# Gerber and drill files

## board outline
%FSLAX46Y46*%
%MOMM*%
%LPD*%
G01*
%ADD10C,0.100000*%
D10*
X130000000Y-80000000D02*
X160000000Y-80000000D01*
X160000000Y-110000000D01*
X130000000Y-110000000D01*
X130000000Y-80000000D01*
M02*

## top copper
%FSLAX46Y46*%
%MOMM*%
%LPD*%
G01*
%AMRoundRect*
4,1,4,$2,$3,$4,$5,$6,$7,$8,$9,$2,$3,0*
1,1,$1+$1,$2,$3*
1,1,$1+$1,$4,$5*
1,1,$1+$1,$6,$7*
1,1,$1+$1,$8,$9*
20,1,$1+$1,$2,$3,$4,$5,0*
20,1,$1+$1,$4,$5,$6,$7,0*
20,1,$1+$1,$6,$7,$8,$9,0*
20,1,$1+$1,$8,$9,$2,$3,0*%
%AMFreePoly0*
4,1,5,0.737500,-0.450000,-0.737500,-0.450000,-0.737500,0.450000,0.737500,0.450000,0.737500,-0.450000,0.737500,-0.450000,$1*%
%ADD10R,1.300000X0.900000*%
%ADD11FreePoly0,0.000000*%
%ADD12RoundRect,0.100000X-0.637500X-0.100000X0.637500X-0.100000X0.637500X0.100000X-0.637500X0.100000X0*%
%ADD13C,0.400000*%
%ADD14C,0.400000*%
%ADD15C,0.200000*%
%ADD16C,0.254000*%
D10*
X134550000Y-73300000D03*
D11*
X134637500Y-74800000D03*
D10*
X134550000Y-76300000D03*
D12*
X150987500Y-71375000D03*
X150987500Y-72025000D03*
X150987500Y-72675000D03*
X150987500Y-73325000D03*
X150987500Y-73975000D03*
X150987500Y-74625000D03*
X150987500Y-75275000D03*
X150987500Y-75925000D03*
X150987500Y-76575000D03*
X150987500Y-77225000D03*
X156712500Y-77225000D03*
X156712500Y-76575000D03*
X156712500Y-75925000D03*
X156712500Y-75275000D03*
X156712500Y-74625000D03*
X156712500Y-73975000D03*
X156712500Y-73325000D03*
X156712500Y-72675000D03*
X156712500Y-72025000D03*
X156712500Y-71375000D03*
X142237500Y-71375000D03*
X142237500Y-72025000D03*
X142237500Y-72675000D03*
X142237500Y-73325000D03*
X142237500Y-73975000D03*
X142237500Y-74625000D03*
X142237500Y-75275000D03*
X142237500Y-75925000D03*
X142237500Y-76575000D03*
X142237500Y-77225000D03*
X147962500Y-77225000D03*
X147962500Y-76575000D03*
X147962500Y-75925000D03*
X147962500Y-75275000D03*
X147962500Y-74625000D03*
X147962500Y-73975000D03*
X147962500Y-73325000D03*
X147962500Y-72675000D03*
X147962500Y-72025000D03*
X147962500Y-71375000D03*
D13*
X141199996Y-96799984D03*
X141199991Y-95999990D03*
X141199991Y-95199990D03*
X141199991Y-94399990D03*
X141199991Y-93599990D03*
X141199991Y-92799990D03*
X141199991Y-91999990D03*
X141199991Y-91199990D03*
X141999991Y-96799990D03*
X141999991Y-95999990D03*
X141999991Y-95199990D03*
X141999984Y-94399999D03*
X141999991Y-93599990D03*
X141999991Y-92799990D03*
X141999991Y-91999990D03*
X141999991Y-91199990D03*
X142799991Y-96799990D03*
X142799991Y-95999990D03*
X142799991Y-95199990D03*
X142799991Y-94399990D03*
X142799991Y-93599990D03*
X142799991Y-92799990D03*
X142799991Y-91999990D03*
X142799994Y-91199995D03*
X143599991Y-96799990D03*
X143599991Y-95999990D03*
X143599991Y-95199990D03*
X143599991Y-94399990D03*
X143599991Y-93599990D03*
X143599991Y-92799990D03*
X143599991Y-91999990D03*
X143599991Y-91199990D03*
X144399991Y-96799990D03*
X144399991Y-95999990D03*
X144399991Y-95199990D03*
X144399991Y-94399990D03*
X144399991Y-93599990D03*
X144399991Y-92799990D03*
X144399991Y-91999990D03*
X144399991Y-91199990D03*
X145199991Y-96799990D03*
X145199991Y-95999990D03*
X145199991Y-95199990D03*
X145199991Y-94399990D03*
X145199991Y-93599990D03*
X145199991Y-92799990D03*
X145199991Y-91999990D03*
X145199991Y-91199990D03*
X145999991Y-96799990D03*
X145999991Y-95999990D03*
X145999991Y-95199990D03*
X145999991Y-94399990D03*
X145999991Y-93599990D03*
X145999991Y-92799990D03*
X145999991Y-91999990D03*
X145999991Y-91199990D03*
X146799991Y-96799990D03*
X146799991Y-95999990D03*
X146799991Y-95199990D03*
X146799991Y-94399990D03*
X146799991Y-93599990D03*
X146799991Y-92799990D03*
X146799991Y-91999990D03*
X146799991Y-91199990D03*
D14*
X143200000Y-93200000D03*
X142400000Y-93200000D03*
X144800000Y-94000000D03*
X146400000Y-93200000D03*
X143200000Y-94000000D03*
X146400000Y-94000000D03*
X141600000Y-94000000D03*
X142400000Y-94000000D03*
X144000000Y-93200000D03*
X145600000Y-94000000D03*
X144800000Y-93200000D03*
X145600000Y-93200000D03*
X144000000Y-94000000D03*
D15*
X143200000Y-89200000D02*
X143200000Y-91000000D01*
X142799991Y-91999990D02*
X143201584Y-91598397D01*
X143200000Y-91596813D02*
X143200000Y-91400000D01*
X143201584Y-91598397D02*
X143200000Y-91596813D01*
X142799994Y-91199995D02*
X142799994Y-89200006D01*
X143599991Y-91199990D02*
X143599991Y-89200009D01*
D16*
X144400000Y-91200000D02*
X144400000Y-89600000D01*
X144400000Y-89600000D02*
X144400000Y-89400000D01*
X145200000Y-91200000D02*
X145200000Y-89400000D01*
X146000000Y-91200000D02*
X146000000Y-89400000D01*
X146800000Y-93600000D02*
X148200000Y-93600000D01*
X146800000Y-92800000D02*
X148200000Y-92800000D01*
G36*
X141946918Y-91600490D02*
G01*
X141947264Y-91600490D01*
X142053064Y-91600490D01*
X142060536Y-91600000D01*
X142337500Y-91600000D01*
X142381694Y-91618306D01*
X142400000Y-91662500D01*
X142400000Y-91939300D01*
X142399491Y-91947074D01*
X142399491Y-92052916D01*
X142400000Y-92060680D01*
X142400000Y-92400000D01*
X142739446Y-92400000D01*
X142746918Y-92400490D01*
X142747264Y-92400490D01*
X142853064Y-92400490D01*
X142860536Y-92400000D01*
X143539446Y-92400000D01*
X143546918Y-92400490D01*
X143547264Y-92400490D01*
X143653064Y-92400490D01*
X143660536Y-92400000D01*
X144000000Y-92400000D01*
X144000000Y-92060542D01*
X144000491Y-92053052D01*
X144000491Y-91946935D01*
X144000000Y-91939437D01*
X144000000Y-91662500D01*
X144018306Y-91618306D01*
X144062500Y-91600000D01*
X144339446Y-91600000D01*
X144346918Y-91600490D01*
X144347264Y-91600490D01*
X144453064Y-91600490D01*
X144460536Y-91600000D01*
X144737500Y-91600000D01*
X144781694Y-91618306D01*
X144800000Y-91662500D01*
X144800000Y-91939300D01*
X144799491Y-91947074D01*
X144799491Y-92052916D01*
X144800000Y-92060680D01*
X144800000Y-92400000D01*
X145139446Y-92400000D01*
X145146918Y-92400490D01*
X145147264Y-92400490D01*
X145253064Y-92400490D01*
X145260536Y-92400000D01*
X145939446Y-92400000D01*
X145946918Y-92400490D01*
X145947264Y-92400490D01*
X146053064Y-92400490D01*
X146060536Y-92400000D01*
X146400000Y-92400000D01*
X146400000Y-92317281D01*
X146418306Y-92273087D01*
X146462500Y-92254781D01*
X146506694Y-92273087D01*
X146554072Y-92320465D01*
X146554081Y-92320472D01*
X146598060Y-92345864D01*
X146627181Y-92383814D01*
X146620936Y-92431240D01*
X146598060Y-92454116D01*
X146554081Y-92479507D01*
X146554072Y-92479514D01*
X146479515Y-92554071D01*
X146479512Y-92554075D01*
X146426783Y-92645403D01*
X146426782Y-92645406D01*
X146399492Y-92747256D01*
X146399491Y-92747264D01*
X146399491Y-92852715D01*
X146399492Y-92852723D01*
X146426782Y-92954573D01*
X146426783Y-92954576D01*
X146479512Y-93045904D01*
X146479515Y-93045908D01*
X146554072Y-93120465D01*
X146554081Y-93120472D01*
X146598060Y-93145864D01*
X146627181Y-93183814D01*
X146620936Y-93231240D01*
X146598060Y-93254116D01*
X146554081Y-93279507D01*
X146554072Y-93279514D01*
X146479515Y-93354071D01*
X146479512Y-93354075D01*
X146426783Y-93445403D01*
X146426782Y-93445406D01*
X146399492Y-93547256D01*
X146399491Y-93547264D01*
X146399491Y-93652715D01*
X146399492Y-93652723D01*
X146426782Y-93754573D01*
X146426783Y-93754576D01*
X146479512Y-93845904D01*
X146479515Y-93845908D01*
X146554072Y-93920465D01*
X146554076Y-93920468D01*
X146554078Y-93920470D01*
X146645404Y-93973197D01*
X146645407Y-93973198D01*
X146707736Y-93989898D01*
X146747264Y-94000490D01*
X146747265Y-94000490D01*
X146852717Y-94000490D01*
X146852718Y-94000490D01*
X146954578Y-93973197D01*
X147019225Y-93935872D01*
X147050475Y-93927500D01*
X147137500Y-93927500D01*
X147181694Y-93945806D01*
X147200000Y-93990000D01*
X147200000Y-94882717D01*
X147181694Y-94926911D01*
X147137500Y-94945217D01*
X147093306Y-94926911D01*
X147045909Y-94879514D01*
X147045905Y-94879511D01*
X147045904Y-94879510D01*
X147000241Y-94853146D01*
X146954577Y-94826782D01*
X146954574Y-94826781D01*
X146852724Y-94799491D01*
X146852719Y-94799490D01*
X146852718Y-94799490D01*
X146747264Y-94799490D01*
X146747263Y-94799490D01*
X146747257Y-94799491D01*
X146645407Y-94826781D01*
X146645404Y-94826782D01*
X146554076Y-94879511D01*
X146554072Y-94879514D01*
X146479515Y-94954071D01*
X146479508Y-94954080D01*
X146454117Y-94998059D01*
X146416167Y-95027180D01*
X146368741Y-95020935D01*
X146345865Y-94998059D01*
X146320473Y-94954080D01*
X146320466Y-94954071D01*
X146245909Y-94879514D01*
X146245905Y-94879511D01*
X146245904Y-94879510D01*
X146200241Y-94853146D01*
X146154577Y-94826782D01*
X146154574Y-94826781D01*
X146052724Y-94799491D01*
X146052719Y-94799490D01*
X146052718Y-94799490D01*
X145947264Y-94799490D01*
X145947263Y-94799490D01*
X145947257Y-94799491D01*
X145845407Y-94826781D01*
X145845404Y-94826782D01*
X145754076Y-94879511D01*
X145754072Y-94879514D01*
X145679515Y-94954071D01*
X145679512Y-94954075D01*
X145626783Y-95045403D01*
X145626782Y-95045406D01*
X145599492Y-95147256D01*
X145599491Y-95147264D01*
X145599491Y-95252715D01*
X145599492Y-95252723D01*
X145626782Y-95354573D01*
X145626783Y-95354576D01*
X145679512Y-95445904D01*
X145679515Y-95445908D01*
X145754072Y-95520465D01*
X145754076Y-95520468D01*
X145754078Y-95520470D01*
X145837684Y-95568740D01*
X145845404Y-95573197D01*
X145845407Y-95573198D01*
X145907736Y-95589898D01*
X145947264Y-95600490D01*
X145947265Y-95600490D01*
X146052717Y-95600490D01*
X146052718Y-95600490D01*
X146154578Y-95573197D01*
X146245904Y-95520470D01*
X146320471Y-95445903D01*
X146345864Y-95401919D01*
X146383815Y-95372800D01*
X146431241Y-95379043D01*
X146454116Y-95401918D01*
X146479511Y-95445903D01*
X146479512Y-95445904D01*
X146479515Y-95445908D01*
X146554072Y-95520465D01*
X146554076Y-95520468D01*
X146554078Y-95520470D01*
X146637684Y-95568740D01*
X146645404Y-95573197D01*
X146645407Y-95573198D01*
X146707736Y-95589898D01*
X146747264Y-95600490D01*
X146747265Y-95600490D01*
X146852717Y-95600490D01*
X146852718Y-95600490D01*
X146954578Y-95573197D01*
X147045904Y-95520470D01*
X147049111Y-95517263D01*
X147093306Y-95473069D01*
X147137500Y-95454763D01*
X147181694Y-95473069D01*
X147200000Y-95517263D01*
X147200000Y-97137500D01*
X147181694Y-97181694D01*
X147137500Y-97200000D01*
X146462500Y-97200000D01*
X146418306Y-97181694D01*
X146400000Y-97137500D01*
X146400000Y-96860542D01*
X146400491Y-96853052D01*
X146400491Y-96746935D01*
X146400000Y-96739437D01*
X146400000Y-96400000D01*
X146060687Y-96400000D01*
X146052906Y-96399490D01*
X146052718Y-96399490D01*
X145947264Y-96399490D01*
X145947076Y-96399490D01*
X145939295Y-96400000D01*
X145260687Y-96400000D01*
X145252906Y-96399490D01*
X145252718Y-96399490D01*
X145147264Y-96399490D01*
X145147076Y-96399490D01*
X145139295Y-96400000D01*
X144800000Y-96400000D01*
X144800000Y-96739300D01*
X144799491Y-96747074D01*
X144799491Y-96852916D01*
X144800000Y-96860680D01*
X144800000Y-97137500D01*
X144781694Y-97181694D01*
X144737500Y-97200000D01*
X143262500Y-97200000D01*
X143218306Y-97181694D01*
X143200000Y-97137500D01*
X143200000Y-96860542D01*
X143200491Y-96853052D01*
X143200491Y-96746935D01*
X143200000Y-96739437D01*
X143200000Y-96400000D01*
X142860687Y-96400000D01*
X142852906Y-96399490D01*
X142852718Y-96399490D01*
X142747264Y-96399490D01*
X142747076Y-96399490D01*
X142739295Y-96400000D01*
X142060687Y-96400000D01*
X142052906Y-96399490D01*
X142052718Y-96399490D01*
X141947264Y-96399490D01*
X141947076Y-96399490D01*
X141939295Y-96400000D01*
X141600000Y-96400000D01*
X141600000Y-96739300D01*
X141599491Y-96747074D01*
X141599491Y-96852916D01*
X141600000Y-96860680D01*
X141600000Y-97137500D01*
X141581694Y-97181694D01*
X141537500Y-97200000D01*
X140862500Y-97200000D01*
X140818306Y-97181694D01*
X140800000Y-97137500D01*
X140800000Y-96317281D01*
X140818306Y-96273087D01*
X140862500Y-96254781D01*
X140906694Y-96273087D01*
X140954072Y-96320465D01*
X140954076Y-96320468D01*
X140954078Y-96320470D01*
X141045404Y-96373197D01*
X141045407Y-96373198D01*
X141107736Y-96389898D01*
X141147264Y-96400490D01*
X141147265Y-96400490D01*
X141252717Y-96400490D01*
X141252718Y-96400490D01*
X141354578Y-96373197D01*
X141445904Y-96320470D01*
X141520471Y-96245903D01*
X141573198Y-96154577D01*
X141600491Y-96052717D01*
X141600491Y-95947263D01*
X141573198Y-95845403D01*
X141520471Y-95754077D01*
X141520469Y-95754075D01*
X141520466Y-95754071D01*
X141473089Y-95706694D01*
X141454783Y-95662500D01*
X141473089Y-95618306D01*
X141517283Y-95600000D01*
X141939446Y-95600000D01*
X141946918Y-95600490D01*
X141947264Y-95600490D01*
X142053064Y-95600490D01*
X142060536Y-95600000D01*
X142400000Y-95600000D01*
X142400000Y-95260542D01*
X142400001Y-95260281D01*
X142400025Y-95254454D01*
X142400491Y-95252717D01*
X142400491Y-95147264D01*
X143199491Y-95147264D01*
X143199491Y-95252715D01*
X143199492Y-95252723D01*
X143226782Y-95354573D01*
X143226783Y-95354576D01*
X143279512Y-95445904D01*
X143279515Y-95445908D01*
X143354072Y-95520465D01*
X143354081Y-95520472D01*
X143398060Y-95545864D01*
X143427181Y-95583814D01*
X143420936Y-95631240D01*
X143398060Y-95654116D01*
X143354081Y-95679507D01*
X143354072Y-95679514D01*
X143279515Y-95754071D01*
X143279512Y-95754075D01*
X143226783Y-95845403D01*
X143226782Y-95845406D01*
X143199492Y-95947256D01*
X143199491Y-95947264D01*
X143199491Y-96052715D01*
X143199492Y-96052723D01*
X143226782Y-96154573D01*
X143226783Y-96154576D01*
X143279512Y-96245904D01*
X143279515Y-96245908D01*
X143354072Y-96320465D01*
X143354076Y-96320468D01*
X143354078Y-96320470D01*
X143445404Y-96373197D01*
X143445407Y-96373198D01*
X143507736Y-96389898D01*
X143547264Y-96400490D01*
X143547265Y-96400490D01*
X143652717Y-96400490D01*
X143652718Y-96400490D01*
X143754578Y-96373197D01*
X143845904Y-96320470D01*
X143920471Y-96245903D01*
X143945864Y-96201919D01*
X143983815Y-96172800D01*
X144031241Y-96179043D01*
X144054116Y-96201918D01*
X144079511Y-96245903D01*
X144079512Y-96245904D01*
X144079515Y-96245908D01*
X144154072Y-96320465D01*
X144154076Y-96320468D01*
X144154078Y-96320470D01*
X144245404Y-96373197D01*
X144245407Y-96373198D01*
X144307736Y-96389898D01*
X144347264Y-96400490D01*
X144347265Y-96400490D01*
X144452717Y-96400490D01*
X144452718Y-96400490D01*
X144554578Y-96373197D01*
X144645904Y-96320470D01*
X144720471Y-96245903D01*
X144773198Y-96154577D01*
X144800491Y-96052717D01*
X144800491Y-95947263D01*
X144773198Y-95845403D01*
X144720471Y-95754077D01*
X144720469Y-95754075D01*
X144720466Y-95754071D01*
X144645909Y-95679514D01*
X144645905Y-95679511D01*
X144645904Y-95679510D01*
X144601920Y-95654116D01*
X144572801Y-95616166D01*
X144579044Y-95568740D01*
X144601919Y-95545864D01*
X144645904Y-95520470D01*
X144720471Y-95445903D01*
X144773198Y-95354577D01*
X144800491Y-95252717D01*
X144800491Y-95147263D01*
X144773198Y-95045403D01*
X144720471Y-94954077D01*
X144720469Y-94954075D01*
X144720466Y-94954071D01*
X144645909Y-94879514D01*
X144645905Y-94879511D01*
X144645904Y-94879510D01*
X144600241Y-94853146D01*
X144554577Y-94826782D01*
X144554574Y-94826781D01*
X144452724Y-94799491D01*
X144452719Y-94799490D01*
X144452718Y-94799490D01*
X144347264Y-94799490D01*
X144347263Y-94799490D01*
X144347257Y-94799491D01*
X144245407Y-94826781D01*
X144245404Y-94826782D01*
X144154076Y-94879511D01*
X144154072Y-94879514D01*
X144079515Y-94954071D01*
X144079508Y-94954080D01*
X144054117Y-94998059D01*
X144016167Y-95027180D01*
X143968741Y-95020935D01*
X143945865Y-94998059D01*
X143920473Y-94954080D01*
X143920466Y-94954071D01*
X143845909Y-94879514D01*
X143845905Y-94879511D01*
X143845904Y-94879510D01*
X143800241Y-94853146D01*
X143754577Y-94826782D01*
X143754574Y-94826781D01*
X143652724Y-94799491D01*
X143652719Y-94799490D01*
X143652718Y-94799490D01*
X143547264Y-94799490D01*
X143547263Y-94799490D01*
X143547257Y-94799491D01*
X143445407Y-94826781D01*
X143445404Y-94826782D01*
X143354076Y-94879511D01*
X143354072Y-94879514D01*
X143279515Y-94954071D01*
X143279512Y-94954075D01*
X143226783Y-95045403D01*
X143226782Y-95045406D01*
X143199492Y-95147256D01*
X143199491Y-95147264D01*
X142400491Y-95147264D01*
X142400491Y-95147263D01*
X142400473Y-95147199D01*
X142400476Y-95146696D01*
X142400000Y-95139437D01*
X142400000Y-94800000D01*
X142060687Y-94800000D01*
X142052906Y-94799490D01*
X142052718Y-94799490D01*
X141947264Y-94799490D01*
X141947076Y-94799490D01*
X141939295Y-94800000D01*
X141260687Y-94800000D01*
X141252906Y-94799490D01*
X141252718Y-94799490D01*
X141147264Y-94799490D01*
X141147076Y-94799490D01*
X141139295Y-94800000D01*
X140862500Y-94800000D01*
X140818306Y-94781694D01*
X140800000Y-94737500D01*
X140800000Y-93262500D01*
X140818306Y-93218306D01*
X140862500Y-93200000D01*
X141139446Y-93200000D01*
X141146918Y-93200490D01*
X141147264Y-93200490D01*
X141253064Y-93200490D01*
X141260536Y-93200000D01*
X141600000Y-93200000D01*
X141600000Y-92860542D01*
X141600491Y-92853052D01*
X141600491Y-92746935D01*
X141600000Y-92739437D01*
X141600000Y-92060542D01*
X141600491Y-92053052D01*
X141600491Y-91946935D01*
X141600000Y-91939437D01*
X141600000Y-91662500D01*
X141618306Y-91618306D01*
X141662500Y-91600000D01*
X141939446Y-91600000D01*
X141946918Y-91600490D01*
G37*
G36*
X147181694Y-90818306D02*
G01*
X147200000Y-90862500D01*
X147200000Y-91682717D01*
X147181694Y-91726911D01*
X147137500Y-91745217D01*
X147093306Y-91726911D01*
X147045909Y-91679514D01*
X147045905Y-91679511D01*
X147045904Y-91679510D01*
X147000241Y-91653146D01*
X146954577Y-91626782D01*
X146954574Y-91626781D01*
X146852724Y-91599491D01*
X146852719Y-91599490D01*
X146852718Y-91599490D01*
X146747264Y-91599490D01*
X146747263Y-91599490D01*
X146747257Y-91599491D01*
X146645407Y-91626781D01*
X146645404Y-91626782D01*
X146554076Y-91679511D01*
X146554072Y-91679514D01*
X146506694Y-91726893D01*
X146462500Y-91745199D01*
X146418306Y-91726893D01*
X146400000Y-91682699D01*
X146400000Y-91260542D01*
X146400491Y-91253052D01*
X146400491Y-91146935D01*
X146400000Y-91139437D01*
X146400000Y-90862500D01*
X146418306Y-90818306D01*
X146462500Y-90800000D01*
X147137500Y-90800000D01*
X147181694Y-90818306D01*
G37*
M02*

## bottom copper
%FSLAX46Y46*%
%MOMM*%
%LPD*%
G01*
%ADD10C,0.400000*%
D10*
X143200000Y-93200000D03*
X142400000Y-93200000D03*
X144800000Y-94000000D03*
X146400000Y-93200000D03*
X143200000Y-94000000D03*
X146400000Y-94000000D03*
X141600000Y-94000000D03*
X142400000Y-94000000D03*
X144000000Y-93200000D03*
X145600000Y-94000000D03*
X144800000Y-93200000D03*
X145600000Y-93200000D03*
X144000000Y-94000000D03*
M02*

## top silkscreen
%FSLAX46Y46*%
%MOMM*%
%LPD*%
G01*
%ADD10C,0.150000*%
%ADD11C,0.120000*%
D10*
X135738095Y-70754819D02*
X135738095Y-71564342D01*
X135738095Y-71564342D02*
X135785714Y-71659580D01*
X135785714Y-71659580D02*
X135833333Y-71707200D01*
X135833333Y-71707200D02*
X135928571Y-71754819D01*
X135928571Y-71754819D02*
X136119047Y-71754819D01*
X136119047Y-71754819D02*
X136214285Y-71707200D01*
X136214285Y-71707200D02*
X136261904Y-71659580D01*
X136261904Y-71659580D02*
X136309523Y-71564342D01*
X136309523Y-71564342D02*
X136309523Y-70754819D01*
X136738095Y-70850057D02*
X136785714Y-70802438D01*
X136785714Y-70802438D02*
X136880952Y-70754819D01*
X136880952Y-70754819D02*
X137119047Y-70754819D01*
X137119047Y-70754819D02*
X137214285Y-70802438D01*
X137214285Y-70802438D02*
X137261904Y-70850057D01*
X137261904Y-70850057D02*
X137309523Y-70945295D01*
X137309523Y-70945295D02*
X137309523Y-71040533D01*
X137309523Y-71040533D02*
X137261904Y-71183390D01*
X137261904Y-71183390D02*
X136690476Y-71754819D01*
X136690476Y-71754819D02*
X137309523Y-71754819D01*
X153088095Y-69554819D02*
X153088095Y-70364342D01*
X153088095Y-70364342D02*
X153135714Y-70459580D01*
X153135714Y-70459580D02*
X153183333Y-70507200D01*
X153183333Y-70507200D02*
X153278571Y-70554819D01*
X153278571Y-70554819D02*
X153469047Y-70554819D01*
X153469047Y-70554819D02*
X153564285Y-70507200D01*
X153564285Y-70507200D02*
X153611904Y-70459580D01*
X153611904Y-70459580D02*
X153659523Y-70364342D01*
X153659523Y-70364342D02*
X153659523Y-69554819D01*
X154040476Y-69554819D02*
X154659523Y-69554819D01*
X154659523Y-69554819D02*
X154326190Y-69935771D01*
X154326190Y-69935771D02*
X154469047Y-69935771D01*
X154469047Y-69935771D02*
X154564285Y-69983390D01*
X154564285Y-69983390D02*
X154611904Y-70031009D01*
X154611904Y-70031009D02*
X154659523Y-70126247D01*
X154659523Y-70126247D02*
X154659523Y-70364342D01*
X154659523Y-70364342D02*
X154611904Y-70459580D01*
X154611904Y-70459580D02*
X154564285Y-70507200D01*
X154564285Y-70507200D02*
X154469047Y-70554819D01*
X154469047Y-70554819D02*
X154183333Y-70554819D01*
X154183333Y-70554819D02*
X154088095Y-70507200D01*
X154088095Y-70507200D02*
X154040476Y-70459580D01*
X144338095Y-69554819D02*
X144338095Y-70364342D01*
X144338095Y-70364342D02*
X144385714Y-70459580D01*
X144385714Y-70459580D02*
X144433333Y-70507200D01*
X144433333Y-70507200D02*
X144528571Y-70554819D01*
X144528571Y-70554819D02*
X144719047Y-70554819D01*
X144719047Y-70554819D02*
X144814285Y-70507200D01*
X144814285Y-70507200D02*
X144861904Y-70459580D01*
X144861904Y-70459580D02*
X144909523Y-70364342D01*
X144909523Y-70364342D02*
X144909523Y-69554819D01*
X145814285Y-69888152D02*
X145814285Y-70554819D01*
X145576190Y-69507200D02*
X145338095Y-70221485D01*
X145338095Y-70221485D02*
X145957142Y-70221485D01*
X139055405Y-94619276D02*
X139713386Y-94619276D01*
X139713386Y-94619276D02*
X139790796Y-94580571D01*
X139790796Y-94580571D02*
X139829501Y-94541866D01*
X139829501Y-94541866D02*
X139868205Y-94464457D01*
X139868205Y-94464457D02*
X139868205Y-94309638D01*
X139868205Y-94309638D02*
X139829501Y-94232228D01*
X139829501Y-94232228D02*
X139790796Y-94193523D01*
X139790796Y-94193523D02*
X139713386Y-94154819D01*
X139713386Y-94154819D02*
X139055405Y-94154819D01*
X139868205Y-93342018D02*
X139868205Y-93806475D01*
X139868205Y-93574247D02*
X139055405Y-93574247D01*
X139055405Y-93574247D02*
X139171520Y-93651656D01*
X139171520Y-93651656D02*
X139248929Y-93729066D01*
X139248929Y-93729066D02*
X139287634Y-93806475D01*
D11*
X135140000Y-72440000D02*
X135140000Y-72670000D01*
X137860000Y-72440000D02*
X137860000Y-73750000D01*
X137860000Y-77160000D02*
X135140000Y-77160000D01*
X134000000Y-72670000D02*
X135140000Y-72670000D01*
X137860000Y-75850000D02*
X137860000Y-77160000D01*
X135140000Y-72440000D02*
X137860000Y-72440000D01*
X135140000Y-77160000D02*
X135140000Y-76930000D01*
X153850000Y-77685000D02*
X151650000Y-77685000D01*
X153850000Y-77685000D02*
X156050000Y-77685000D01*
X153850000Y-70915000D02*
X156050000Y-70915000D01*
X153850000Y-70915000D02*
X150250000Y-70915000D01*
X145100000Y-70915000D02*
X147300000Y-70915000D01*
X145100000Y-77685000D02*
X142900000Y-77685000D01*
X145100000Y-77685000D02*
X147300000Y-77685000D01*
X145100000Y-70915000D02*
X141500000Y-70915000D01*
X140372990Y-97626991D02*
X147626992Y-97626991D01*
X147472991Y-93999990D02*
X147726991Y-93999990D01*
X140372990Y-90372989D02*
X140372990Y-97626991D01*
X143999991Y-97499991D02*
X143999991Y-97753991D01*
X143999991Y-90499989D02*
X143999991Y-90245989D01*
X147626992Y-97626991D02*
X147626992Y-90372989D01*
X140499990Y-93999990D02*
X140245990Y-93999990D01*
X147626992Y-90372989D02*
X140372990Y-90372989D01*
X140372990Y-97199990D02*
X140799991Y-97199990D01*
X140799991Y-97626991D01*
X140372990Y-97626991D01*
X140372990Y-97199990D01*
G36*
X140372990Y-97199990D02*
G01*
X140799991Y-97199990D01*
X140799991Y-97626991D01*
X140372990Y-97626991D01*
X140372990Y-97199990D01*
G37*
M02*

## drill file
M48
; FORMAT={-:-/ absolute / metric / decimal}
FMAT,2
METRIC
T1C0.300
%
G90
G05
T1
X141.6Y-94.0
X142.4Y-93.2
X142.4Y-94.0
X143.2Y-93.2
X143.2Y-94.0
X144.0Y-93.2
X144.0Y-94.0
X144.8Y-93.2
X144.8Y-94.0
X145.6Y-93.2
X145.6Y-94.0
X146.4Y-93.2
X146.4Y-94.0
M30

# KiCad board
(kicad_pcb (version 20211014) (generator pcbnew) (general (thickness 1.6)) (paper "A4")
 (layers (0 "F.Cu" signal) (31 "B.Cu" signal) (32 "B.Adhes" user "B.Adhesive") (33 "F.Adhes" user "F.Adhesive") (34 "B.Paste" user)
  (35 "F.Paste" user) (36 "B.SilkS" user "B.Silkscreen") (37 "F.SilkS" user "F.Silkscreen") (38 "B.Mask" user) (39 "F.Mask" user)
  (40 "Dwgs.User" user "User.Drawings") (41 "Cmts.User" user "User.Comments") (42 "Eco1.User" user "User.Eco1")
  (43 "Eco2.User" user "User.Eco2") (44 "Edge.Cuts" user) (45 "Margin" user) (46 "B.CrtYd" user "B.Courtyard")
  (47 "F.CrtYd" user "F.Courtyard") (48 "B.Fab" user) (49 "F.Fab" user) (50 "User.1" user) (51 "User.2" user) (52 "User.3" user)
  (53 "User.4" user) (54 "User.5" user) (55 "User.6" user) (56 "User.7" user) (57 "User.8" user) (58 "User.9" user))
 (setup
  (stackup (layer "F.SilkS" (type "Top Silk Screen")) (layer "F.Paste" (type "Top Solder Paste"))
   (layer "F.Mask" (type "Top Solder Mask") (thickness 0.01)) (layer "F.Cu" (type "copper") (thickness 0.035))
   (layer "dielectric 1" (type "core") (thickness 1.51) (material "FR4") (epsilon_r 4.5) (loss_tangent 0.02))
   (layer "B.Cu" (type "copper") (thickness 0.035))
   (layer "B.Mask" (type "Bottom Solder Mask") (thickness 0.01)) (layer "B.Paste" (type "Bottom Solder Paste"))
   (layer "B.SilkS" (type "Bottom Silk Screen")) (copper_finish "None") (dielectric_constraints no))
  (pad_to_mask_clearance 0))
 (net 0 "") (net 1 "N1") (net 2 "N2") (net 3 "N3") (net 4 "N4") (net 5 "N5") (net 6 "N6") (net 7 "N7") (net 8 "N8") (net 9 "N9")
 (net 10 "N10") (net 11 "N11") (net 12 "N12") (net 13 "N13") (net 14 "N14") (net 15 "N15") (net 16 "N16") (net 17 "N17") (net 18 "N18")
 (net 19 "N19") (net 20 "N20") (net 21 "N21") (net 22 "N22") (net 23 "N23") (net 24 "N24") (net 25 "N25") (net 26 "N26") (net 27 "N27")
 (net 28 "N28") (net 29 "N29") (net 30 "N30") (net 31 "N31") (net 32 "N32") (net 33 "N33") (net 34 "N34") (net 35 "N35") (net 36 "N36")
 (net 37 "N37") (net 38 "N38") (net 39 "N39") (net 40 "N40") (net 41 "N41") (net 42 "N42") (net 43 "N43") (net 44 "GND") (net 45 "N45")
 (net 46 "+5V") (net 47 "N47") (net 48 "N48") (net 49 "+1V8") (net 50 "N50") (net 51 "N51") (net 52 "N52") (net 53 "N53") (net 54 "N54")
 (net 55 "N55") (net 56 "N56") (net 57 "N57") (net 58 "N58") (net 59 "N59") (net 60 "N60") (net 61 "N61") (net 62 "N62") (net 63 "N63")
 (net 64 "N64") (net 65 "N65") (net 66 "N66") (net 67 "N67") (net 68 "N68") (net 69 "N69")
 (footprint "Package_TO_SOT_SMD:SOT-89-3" (layer "F.Cu") (at 136.2 74.8)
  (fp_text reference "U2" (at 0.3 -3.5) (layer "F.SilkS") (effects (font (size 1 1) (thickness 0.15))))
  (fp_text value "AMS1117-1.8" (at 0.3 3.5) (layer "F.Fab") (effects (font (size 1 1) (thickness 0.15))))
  (fp_line (start -1.06 -2.36) (end -1.06 -2.13) (layer "F.SilkS") (width 0.12))
  (fp_line (start 1.66 -2.36) (end 1.66 -1.05) (layer "F.SilkS") (width 0.12))
  (fp_line (start 1.66 2.36) (end -1.06 2.36) (layer "F.SilkS") (width 0.12))
  (fp_line (start -2.2 -2.13) (end -1.06 -2.13) (layer "F.SilkS") (width 0.12))
  (fp_line (start 1.66 1.05) (end 1.66 2.36) (layer "F.SilkS") (width 0.12))
  (fp_line (start -1.06 -2.36) (end 1.66 -2.36) (layer "F.SilkS") (width 0.12))
  (fp_line (start -1.06 2.36) (end -1.06 2.13) (layer "F.SilkS") (width 0.12))
  (pad "1" smd rect locked (at -1.65 -1.5) (size 1.3 0.9) (layers "F.Cu" "F.Paste" "F.Mask") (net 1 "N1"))
  (pad "2" smd custom locked (at -1.5625 0) (size 1.475 0.9) (layers "F.Cu" "F.Paste" "F.Mask") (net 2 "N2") (zone_connect 2)
   (options (clearance outline) (anchor rect)) (primitives))
  (pad "3" smd rect locked (at -1.65 1.5) (size 1.3 0.9) (layers "F.Cu" "F.Paste" "F.Mask") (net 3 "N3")))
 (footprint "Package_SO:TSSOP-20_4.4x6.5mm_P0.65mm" (layer "F.Cu") (at 153.85 74.3)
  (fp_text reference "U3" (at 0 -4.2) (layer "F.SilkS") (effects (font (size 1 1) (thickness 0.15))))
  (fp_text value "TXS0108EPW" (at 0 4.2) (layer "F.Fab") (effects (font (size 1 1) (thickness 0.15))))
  (fp_line (start 0 3.385) (end -2.2 3.385) (layer "F.SilkS") (width 0.12))
  (fp_line (start 0 3.385) (end 2.2 3.385) (layer "F.SilkS") (width 0.12))
  (fp_line (start 0 -3.385) (end 2.2 -3.385) (layer "F.SilkS") (width 0.12))
  (fp_line (start 0 -3.385) (end -3.6 -3.385) (layer "F.SilkS") (width 0.12))
  (pad "1" smd roundrect locked (at -2.8625 -2.925) (size 1.475 0.4) (layers "F.Cu" "F.Paste" "F.Mask") (roundrect_rratio 0.25) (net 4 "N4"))
  (pad "2" smd roundrect locked (at -2.8625 -2.275) (size 1.475 0.4) (layers "F.Cu" "F.Paste" "F.Mask") (roundrect_rratio 0.25) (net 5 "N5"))
  (pad "3" smd roundrect locked (at -2.8625 -1.625) (size 1.475 0.4) (layers "F.Cu" "F.Paste" "F.Mask") (roundrect_rratio 0.25) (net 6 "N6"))
  (pad "4" smd roundrect locked (at -2.8625 -0.975) (size 1.475 0.4) (layers "F.Cu" "F.Paste" "F.Mask") (roundrect_rratio 0.25) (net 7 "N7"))
  (pad "5" smd roundrect locked (at -2.8625 -0.325) (size 1.475 0.4) (layers "F.Cu" "F.Paste" "F.Mask") (roundrect_rratio 0.25) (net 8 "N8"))
  (pad "6" smd roundrect locked (at -2.8625 0.325) (size 1.475 0.4) (layers "F.Cu" "F.Paste" "F.Mask") (roundrect_rratio 0.25) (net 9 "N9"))
  (pad "7" smd roundrect locked (at -2.8625 0.975) (size 1.475 0.4) (layers "F.Cu" "F.Paste" "F.Mask") (roundrect_rratio 0.25)
   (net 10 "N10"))
  (pad "8" smd roundrect locked (at -2.8625 1.625) (size 1.475 0.4) (layers "F.Cu" "F.Paste" "F.Mask") (roundrect_rratio 0.25)
   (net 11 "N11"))
  (pad "9" smd roundrect locked (at -2.8625 2.275) (size 1.475 0.4) (layers "F.Cu" "F.Paste" "F.Mask") (roundrect_rratio 0.25)
   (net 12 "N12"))
  (pad "10" smd roundrect locked (at -2.8625 2.925) (size 1.475 0.4) (layers "F.Cu" "F.Paste" "F.Mask") (roundrect_rratio 0.25)
   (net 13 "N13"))
  (pad "11" smd roundrect locked (at 2.8625 2.925) (size 1.475 0.4) (layers "F.Cu" "F.Paste" "F.Mask") (roundrect_rratio 0.25)
   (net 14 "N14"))
  (pad "12" smd roundrect locked (at 2.8625 2.275) (size 1.475 0.4) (layers "F.Cu" "F.Paste" "F.Mask") (roundrect_rratio 0.25)
   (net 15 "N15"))
  (pad "13" smd roundrect locked (at 2.8625 1.625) (size 1.475 0.4) (layers "F.Cu" "F.Paste" "F.Mask") (roundrect_rratio 0.25)
   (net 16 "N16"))
  (pad "14" smd roundrect locked (at 2.8625 0.975) (size 1.475 0.4) (layers "F.Cu" "F.Paste" "F.Mask") (roundrect_rratio 0.25)
   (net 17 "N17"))
  (pad "15" smd roundrect locked (at 2.8625 0.325) (size 1.475 0.4) (layers "F.Cu" "F.Paste" "F.Mask") (roundrect_rratio 0.25)
   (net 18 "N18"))
  (pad "16" smd roundrect locked (at 2.8625 -0.325) (size 1.475 0.4) (layers "F.Cu" "F.Paste" "F.Mask") (roundrect_rratio 0.25)
   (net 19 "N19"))
  (pad "17" smd roundrect locked (at 2.8625 -0.975) (size 1.475 0.4) (layers "F.Cu" "F.Paste" "F.Mask") (roundrect_rratio 0.25)
   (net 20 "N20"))
  (pad "18" smd roundrect locked (at 2.8625 -1.625) (size 1.475 0.4) (layers "F.Cu" "F.Paste" "F.Mask") (roundrect_rratio 0.25)
   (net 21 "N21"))
  (pad "19" smd roundrect locked (at 2.8625 -2.275) (size 1.475 0.4) (layers "F.Cu" "F.Paste" "F.Mask") (roundrect_rratio 0.25)
   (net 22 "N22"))
  (pad "20" smd roundrect locked (at 2.8625 -2.925) (size 1.475 0.4) (layers "F.Cu" "F.Paste" "F.Mask") (roundrect_rratio 0.25)
   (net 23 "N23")))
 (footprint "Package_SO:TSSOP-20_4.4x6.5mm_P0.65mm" (layer "F.Cu") (at 145.1 74.3)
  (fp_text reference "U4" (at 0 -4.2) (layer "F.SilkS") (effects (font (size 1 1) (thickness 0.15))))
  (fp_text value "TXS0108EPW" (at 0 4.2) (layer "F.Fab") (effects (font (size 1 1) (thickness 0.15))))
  (fp_line (start 0 -3.385) (end 2.2 -3.385) (layer "F.SilkS") (width 0.12))
  (fp_line (start 0 3.385) (end -2.2 3.385) (layer "F.SilkS") (width 0.12))
  (fp_line (start 0 3.385) (end 2.2 3.385) (layer "F.SilkS") (width 0.12))
  (fp_line (start 0 -3.385) (end -3.6 -3.385) (layer "F.SilkS") (width 0.12))
  (pad "1" smd roundrect locked (at -2.8625 -2.925) (size 1.475 0.4) (layers "F.Cu" "F.Paste" "F.Mask") (roundrect_rratio 0.25)
   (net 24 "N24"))
  (pad "2" smd roundrect locked (at -2.8625 -2.275) (size 1.475 0.4) (layers "F.Cu" "F.Paste" "F.Mask") (roundrect_rratio 0.25)
   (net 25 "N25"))
  (pad "3" smd roundrect locked (at -2.8625 -1.625) (size 1.475 0.4) (layers "F.Cu" "F.Paste" "F.Mask") (roundrect_rratio 0.25)
   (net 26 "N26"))
  (pad "4" smd roundrect locked (at -2.8625 -0.975) (size 1.475 0.4) (layers "F.Cu" "F.Paste" "F.Mask") (roundrect_rratio 0.25)
   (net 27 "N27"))
  (pad "5" smd roundrect locked (at -2.8625 -0.325) (size 1.475 0.4) (layers "F.Cu" "F.Paste" "F.Mask") (roundrect_rratio 0.25)
   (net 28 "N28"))
  (pad "6" smd roundrect locked (at -2.8625 0.325) (size 1.475 0.4) (layers "F.Cu" "F.Paste" "F.Mask") (roundrect_rratio 0.25)
   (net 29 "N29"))
  (pad "7" smd roundrect locked (at -2.8625 0.975) (size 1.475 0.4) (layers "F.Cu" "F.Paste" "F.Mask") (roundrect_rratio 0.25)
   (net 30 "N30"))
  (pad "8" smd roundrect locked (at -2.8625 1.625) (size 1.475 0.4) (layers "F.Cu" "F.Paste" "F.Mask") (roundrect_rratio 0.25)
   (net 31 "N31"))
  (pad "9" smd roundrect locked (at -2.8625 2.275) (size 1.475 0.4) (layers "F.Cu" "F.Paste" "F.Mask") (roundrect_rratio 0.25)
   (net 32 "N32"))
  (pad "10" smd roundrect locked (at -2.8625 2.925) (size 1.475 0.4) (layers "F.Cu" "F.Paste" "F.Mask") (roundrect_rratio 0.25)
   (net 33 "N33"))
  (pad "11" smd roundrect locked (at 2.8625 2.925) (size 1.475 0.4) (layers "F.Cu" "F.Paste" "F.Mask") (roundrect_rratio 0.25)
   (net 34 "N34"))
  (pad "12" smd roundrect locked (at 2.8625 2.275) (size 1.475 0.4) (layers "F.Cu" "F.Paste" "F.Mask") (roundrect_rratio 0.25)
   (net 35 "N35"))
  (pad "13" smd roundrect locked (at 2.8625 1.625) (size 1.475 0.4) (layers "F.Cu" "F.Paste" "F.Mask") (roundrect_rratio 0.25)
   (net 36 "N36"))
  (pad "14" smd roundrect locked (at 2.8625 0.975) (size 1.475 0.4) (layers "F.Cu" "F.Paste" "F.Mask") (roundrect_rratio 0.25)
   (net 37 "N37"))
  (pad "15" smd roundrect locked (at 2.8625 0.325) (size 1.475 0.4) (layers "F.Cu" "F.Paste" "F.Mask") (roundrect_rratio 0.25)
   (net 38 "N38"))
  (pad "16" smd roundrect locked (at 2.8625 -0.325) (size 1.475 0.4) (layers "F.Cu" "F.Paste" "F.Mask") (roundrect_rratio 0.25)
   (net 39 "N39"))
  (pad "17" smd roundrect locked (at 2.8625 -0.975) (size 1.475 0.4) (layers "F.Cu" "F.Paste" "F.Mask") (roundrect_rratio 0.25)
   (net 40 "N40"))
  (pad "18" smd roundrect locked (at 2.8625 -1.625) (size 1.475 0.4) (layers "F.Cu" "F.Paste" "F.Mask") (roundrect_rratio 0.25)
   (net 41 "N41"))
  (pad "19" smd roundrect locked (at 2.8625 -2.275) (size 1.475 0.4) (layers "F.Cu" "F.Paste" "F.Mask") (roundrect_rratio 0.25)
   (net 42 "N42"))
  (pad "20" smd roundrect locked (at 2.8625 -2.925) (size 1.475 0.4) (layers "F.Cu" "F.Paste" "F.Mask") (roundrect_rratio 0.25)
   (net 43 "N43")))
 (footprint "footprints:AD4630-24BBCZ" (layer "F.Cu") (at 143.999991 93.99999 90)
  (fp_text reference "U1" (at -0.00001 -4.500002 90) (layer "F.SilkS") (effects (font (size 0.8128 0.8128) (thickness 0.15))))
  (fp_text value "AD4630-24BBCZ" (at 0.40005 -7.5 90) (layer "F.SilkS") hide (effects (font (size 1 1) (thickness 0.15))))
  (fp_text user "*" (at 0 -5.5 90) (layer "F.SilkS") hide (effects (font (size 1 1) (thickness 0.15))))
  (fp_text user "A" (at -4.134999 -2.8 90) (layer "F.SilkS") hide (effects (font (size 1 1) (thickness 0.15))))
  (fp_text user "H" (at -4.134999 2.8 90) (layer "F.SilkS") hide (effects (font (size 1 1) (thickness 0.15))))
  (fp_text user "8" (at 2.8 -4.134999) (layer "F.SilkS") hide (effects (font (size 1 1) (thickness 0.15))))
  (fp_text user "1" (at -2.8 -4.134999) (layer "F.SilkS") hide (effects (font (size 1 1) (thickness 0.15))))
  (fp_line (start -3.627001 -3.627001) (end -3.627001 3.627001) (layer "F.SilkS") (width 0.12))
  (fp_line (start 0 3.473) (end 0 3.727) (layer "F.SilkS") (width 0.12))
  (fp_line (start 3.627001 -3.627001) (end -3.627001 -3.627001) (layer "F.SilkS") (width 0.12))
  (fp_line (start -3.500001 0) (end -3.754001 0) (layer "F.SilkS") (width 0.12))
  (fp_line (start 3.500001 0) (end 3.754001 0) (layer "F.SilkS") (width 0.12))
  (fp_line (start -3.627001 3.627001) (end 3.627001 3.627001) (layer "F.SilkS") (width 0.12))
  (fp_line (start 0 -3.500001) (end 0 -3.754001) (layer "F.SilkS") (width 0.12))
  (fp_line (start 3.627001 3.627001) (end 3.627001 -3.627001) (layer "F.SilkS") (width 0.12))
  (fp_rect (start -3.627001 -3.627001) (end -3.2 -3.2) (layer "F.SilkS") (width 0.12) (fill solid))
  (pad "A1" smd circle (at -2.799994 -2.799995 90) (size 0.4 0.4) (layers "F.Cu" "F.Paste" "F.Mask") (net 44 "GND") (clearance 0.127))
  (pad "A2" smd circle (at -2 -2.8 90) (size 0.4 0.4) (layers "F.Cu" "F.Paste" "F.Mask") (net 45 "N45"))
  (pad "A3" smd circle (at -1.2 -2.8 90) (size 0.4 0.4) (layers "F.Cu" "F.Paste" "F.Mask") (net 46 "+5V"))
  (pad "A4" smd circle (at -0.4 -2.8 90) (size 0.4 0.4) (layers "F.Cu" "F.Paste" "F.Mask") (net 44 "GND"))
  (pad "A5" smd circle (at 0.4 -2.8 90) (size 0.4 0.4) (layers "F.Cu" "F.Paste" "F.Mask") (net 44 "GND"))
  (pad "A6" smd circle (at 1.2 -2.8 90) (size 0.4 0.4) (layers "F.Cu" "F.Paste" "F.Mask") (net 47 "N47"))
  (pad "A7" smd circle (at 2 -2.8 90) (size 0.4 0.4) (layers "F.Cu" "F.Paste" "F.Mask") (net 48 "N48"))
  (pad "A8" smd circle (at 2.8 -2.8 90) (size 0.4 0.4) (layers "F.Cu" "F.Paste" "F.Mask") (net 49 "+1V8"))
  (pad "B1" smd circle (at -2.8 -2 90) (size 0.4 0.4) (layers "F.Cu" "F.Paste" "F.Mask") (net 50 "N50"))
  (pad "B2" smd circle (at -2 -2 90) (size 0.4 0.4) (layers "F.Cu" "F.Paste" "F.Mask") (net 44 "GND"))
  (pad "B3" smd circle (at -1.2 -2 90) (size 0.4 0.4) (layers "F.Cu" "F.Paste" "F.Mask") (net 46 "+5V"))
  (pad "B4" smd circle (at -0.400009 -2.000007 90) (size 0.4 0.4) (layers "F.Cu" "F.Paste" "F.Mask") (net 44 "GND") (clearance 0.127))
  (pad "B5" smd circle (at 0.4 -2 90) (size 0.4 0.4) (layers "F.Cu" "F.Paste" "F.Mask") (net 44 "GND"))
  (pad "B6" smd circle (at 1.2 -2 90) (size 0.4 0.4) (layers "F.Cu" "F.Paste" "F.Mask") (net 44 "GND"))
  (pad "B7" smd circle (at 2 -2 90) (size 0.4 0.4) (layers "F.Cu" "F.Paste" "F.Mask") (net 44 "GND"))
  (pad "B8" smd circle (at 2.8 -2 90) (size 0.4 0.4) (layers "F.Cu" "F.Paste" "F.Mask") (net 46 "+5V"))
  (pad "C1" smd circle (at -2.8 -1.2 90) (size 0.4 0.4) (layers "F.Cu" "F.Paste" "F.Mask") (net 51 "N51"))
  (pad "C2" smd circle (at -2 -1.2 90) (size 0.4 0.4) (layers "F.Cu" "F.Paste" "F.Mask") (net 44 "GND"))
  (pad "C3" smd circle (at -1.2 -1.2 90) (size 0.4 0.4) (layers "F.Cu" "F.Paste" "F.Mask") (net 44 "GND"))
  (pad "C4" smd circle (at -0.4 -1.2 90) (size 0.4 0.4) (layers "F.Cu" "F.Paste" "F.Mask") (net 44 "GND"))
  (pad "C5" smd circle (at 0.4 -1.2 90) (size 0.4 0.4) (layers "F.Cu" "F.Paste" "F.Mask") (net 44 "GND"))
  (pad "C6" smd circle (at 1.2 -1.2 90) (size 0.4 0.4) (layers "F.Cu" "F.Paste" "F.Mask") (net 44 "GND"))
  (pad "C7" smd circle (at 2 -1.2 90) (size 0.4 0.4) (layers "F.Cu" "F.Paste" "F.Mask") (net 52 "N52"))
  (pad "C8" smd circle (at 2.799995 -1.199997 90) (size 0.4 0.4) (layers "F.Cu" "F.Paste" "F.Mask") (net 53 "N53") (clearance 0.00254))
  (pad "D1" smd circle (at -2.8 -0.4 90) (size 0.4 0.4) (layers "F.Cu" "F.Paste" "F.Mask") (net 44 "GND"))
  (pad "D2" smd circle (at -2 -0.4 90) (size 0.4 0.4) (layers "F.Cu" "F.Paste" "F.Mask") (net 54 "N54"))
  (pad "D3" smd circle (at -1.2 -0.4 90) (size 0.4 0.4) (layers "F.Cu" "F.Paste" "F.Mask") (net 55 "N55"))
  (pad "D4" smd circle (at -0.4 -0.4 90) (size 0.4 0.4) (layers "F.Cu" "F.Paste" "F.Mask") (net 44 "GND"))
  (pad "D5" smd circle (at 0.4 -0.4 90) (size 0.4 0.4) (layers "F.Cu" "F.Paste" "F.Mask") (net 44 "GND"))
  (pad "D6" smd circle (at 1.2 -0.4 90) (size 0.4 0.4) (layers "F.Cu" "F.Paste" "F.Mask") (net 44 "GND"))
  (pad "D7" smd circle (at 2 -0.4 90) (size 0.4 0.4) (layers "F.Cu" "F.Paste" "F.Mask") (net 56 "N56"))
  (pad "D8" smd circle (at 2.8 -0.4 90) (size 0.4 0.4) (layers "F.Cu" "F.Paste" "F.Mask") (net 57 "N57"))
  (pad "E1" smd circle (at -2.8 0.4 90) (size 0.4 0.4) (layers "F.Cu" "F.Paste" "F.Mask") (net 44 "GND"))
  (pad "E2" smd circle (at -2 0.4 90) (size 0.4 0.4) (layers "F.Cu" "F.Paste" "F.Mask") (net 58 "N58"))
  (pad "E3" smd circle (at -1.2 0.4 90) (size 0.4 0.4) (layers "F.Cu" "F.Paste" "F.Mask") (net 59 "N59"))
  (pad "E4" smd circle (at -0.4 0.4 90) (size 0.4 0.4) (layers "F.Cu" "F.Paste" "F.Mask") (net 44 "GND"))
  (pad "E5" smd circle (at 0.4 0.4 90) (size 0.4 0.4) (layers "F.Cu" "F.Paste" "F.Mask") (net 44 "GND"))
  (pad "E6" smd circle (at 1.2 0.4 90) (size 0.4 0.4) (layers "F.Cu" "F.Paste" "F.Mask") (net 44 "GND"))
  (pad "E7" smd circle (at 2 0.4 90) (size 0.4 0.4) (layers "F.Cu" "F.Paste" "F.Mask") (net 44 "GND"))
  (pad "E8" smd circle (at 2.8 0.4 90) (size 0.4 0.4) (layers "F.Cu" "F.Paste" "F.Mask") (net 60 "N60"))
  (pad "F1" smd circle (at -2.8 1.2 90) (size 0.4 0.4) (layers "F.Cu" "F.Paste" "F.Mask") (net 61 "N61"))
  (pad "F2" smd circle (at -2 1.2 90) (size 0.4 0.4) (layers "F.Cu" "F.Paste" "F.Mask") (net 44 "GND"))
  (pad "F3" smd circle (at -1.2 1.2 90) (size 0.4 0.4) (layers "F.Cu" "F.Paste" "F.Mask") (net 44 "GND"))
  (pad "F4" smd circle (at -0.4 1.2 90) (size 0.4 0.4) (layers "F.Cu" "F.Paste" "F.Mask") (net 44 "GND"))
  (pad "F5" smd circle (at 0.4 1.2 90) (size 0.4 0.4) (layers "F.Cu" "F.Paste" "F.Mask") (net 44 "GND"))
  (pad "F6" smd circle (at 1.2 1.2 90) (size 0.4 0.4) (layers "F.Cu" "F.Paste" "F.Mask") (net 44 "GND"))
  (pad "F7" smd circle (at 2 1.2 90) (size 0.4 0.4) (layers "F.Cu" "F.Paste" "F.Mask") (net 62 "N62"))
  (pad "F8" smd circle (at 2.8 1.2 90) (size 0.4 0.4) (layers "F.Cu" "F.Paste" "F.Mask") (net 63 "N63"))
  (pad "G1" smd circle (at -2.8 2 90) (size 0.4 0.4) (layers "F.Cu" "F.Paste" "F.Mask") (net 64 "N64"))
  (pad "G2" smd circle (at -2 2 90) (size 0.4 0.4) (layers "F.Cu" "F.Paste" "F.Mask") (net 44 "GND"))
  (pad "G3" smd circle (at -1.2 2 90) (size 0.4 0.4) (layers "F.Cu" "F.Paste" "F.Mask") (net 49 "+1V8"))
  (pad "G4" smd circle (at -0.4 2 90) (size 0.4 0.4) (layers "F.Cu" "F.Paste" "F.Mask") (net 44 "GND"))
  (pad "G5" smd circle (at 0.4 2 90) (size 0.4 0.4) (layers "F.Cu" "F.Paste" "F.Mask") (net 44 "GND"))
  (pad "G6" smd circle (at 1.2 2 90) (size 0.4 0.4) (layers "F.Cu" "F.Paste" "F.Mask") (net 44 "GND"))
  (pad "G7" smd circle (at 2 2 90) (size 0.4 0.4) (layers "F.Cu" "F.Paste" "F.Mask") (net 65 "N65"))
  (pad "G8" smd circle (at 2.8 2 90) (size 0.4 0.4) (layers "F.Cu" "F.Paste" "F.Mask") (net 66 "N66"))
  (pad "H1" smd circle (at -2.8 2.8 90) (size 0.4 0.4) (layers "F.Cu" "F.Paste" "F.Mask") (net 44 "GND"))
  (pad "H2" smd circle (at -2 2.8 90) (size 0.4 0.4) (layers "F.Cu" "F.Paste" "F.Mask") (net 44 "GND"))
  (pad "H3" smd circle (at -1.2 2.8 90) (size 0.4 0.4) (layers "F.Cu" "F.Paste" "F.Mask") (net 49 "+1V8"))
  (pad "H4" smd circle (at -0.4 2.8 90) (size 0.4 0.4) (layers "F.Cu" "F.Paste" "F.Mask") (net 44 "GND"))
  (pad "H5" smd circle (at 0.4 2.8 90) (size 0.4 0.4) (layers "F.Cu" "F.Paste" "F.Mask") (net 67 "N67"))
  (pad "H6" smd circle (at 1.2 2.8 90) (size 0.4 0.4) (layers "F.Cu" "F.Paste" "F.Mask") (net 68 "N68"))
  (pad "H7" smd circle (at 2 2.8 90) (size 0.4 0.4) (layers "F.Cu" "F.Paste" "F.Mask") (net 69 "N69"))
  (pad "H8" smd circle (at 2.8 2.8 90) (size 0.4 0.4) (layers "F.Cu" "F.Paste" "F.Mask") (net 44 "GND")))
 (gr_rect (start 130 80) (end 160 110) (layer "Edge.Cuts") (width 0.1) (fill none))
 (segment (start 143.2 89.2) (end 143.2 91) (width 0.2) (layer "F.Cu") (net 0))
 (via (at 143.2 93.2) (size 0.4) (drill 0.3) (layers "F.Cu" "B.Cu") (free) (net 44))
 (via (at 142.4 93.2) (size 0.4) (drill 0.3) (layers "F.Cu" "B.Cu") (free) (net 44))
 (via (at 144.8 94) (size 0.4) (drill 0.3) (layers "F.Cu" "B.Cu") (free) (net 44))
 (via (at 146.4 93.2) (size 0.4) (drill 0.3) (layers "F.Cu" "B.Cu") (free) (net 44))
 (via (at 143.2 94) (size 0.4) (drill 0.3) (layers "F.Cu" "B.Cu") (free) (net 44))
 (via (at 146.4 94) (size 0.4) (drill 0.3) (layers "F.Cu" "B.Cu") (free) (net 44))
 (via (at 141.6 94) (size 0.4) (drill 0.3) (layers "F.Cu" "B.Cu") (free) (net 44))
 (via (at 142.4 94) (size 0.4) (drill 0.3) (layers "F.Cu" "B.Cu") (free) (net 44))
 (via (at 144 93.2) (size 0.4) (drill 0.3) (layers "F.Cu" "B.Cu") (free) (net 44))
 (via (at 145.6 94) (size 0.4) (drill 0.3) (layers "F.Cu" "B.Cu") (free) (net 44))
 (via (at 144.8 93.2) (size 0.4) (drill 0.3) (layers "F.Cu" "B.Cu") (free) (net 44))
 (via (at 145.6 93.2) (size 0.4) (drill 0.3) (layers "F.Cu" "B.Cu") (free) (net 44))
 (via (at 144 94) (size 0.4) (drill 0.3) (layers "F.Cu" "B.Cu") (free) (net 44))
 (segment (start 142.799991 91.99999) (end 143.201584 91.598397) (width 0.2) (layer "F.Cu") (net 52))
 (segment (start 143.2 91.596813) (end 143.2 91.4) (width 0.2) (layer "F.Cu") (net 52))
 (segment (start 143.201584 91.598397) (end 143.2 91.596813) (width 0.2) (layer "F.Cu") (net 52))
 (segment (start 142.799994 91.199995) (end 142.799994 89.200006) (width 0.2) (layer "F.Cu") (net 53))
 (segment (start 143.599991 91.19999) (end 143.599991 89.200009) (width 0.2) (layer "F.Cu") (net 57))
 (segment (start 144.4 91.2) (end 144.4 89.6) (width 0.254) (layer "F.Cu") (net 60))
 (segment (start 144.4 89.6) (end 144.4 89.4) (width 0.254) (layer "F.Cu") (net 60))
 (segment (start 145.2 91.2) (end 145.2 89.4) (width 0.254) (layer "F.Cu") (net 63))
 (segment (start 146 91.2) (end 146 89.4) (width 0.254) (layer "F.Cu") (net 66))
 (segment (start 146.8 93.6) (end 148.2 93.6) (width 0.254) (layer "F.Cu") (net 67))
 (segment (start 146.8 92.8) (end 148.2 92.8) (width 0.254) (layer "F.Cu") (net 68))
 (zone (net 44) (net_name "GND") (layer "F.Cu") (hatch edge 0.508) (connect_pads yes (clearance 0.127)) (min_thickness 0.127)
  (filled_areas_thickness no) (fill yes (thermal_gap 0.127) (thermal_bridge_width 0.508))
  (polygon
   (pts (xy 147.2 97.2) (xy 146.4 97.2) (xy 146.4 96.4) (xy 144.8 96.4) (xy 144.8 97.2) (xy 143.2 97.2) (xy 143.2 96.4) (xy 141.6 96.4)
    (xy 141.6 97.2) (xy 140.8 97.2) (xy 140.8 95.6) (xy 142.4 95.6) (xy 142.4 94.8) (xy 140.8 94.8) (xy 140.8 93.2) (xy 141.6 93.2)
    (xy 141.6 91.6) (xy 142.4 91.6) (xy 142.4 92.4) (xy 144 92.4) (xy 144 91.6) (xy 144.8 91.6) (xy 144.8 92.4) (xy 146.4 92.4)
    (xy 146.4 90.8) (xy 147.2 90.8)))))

